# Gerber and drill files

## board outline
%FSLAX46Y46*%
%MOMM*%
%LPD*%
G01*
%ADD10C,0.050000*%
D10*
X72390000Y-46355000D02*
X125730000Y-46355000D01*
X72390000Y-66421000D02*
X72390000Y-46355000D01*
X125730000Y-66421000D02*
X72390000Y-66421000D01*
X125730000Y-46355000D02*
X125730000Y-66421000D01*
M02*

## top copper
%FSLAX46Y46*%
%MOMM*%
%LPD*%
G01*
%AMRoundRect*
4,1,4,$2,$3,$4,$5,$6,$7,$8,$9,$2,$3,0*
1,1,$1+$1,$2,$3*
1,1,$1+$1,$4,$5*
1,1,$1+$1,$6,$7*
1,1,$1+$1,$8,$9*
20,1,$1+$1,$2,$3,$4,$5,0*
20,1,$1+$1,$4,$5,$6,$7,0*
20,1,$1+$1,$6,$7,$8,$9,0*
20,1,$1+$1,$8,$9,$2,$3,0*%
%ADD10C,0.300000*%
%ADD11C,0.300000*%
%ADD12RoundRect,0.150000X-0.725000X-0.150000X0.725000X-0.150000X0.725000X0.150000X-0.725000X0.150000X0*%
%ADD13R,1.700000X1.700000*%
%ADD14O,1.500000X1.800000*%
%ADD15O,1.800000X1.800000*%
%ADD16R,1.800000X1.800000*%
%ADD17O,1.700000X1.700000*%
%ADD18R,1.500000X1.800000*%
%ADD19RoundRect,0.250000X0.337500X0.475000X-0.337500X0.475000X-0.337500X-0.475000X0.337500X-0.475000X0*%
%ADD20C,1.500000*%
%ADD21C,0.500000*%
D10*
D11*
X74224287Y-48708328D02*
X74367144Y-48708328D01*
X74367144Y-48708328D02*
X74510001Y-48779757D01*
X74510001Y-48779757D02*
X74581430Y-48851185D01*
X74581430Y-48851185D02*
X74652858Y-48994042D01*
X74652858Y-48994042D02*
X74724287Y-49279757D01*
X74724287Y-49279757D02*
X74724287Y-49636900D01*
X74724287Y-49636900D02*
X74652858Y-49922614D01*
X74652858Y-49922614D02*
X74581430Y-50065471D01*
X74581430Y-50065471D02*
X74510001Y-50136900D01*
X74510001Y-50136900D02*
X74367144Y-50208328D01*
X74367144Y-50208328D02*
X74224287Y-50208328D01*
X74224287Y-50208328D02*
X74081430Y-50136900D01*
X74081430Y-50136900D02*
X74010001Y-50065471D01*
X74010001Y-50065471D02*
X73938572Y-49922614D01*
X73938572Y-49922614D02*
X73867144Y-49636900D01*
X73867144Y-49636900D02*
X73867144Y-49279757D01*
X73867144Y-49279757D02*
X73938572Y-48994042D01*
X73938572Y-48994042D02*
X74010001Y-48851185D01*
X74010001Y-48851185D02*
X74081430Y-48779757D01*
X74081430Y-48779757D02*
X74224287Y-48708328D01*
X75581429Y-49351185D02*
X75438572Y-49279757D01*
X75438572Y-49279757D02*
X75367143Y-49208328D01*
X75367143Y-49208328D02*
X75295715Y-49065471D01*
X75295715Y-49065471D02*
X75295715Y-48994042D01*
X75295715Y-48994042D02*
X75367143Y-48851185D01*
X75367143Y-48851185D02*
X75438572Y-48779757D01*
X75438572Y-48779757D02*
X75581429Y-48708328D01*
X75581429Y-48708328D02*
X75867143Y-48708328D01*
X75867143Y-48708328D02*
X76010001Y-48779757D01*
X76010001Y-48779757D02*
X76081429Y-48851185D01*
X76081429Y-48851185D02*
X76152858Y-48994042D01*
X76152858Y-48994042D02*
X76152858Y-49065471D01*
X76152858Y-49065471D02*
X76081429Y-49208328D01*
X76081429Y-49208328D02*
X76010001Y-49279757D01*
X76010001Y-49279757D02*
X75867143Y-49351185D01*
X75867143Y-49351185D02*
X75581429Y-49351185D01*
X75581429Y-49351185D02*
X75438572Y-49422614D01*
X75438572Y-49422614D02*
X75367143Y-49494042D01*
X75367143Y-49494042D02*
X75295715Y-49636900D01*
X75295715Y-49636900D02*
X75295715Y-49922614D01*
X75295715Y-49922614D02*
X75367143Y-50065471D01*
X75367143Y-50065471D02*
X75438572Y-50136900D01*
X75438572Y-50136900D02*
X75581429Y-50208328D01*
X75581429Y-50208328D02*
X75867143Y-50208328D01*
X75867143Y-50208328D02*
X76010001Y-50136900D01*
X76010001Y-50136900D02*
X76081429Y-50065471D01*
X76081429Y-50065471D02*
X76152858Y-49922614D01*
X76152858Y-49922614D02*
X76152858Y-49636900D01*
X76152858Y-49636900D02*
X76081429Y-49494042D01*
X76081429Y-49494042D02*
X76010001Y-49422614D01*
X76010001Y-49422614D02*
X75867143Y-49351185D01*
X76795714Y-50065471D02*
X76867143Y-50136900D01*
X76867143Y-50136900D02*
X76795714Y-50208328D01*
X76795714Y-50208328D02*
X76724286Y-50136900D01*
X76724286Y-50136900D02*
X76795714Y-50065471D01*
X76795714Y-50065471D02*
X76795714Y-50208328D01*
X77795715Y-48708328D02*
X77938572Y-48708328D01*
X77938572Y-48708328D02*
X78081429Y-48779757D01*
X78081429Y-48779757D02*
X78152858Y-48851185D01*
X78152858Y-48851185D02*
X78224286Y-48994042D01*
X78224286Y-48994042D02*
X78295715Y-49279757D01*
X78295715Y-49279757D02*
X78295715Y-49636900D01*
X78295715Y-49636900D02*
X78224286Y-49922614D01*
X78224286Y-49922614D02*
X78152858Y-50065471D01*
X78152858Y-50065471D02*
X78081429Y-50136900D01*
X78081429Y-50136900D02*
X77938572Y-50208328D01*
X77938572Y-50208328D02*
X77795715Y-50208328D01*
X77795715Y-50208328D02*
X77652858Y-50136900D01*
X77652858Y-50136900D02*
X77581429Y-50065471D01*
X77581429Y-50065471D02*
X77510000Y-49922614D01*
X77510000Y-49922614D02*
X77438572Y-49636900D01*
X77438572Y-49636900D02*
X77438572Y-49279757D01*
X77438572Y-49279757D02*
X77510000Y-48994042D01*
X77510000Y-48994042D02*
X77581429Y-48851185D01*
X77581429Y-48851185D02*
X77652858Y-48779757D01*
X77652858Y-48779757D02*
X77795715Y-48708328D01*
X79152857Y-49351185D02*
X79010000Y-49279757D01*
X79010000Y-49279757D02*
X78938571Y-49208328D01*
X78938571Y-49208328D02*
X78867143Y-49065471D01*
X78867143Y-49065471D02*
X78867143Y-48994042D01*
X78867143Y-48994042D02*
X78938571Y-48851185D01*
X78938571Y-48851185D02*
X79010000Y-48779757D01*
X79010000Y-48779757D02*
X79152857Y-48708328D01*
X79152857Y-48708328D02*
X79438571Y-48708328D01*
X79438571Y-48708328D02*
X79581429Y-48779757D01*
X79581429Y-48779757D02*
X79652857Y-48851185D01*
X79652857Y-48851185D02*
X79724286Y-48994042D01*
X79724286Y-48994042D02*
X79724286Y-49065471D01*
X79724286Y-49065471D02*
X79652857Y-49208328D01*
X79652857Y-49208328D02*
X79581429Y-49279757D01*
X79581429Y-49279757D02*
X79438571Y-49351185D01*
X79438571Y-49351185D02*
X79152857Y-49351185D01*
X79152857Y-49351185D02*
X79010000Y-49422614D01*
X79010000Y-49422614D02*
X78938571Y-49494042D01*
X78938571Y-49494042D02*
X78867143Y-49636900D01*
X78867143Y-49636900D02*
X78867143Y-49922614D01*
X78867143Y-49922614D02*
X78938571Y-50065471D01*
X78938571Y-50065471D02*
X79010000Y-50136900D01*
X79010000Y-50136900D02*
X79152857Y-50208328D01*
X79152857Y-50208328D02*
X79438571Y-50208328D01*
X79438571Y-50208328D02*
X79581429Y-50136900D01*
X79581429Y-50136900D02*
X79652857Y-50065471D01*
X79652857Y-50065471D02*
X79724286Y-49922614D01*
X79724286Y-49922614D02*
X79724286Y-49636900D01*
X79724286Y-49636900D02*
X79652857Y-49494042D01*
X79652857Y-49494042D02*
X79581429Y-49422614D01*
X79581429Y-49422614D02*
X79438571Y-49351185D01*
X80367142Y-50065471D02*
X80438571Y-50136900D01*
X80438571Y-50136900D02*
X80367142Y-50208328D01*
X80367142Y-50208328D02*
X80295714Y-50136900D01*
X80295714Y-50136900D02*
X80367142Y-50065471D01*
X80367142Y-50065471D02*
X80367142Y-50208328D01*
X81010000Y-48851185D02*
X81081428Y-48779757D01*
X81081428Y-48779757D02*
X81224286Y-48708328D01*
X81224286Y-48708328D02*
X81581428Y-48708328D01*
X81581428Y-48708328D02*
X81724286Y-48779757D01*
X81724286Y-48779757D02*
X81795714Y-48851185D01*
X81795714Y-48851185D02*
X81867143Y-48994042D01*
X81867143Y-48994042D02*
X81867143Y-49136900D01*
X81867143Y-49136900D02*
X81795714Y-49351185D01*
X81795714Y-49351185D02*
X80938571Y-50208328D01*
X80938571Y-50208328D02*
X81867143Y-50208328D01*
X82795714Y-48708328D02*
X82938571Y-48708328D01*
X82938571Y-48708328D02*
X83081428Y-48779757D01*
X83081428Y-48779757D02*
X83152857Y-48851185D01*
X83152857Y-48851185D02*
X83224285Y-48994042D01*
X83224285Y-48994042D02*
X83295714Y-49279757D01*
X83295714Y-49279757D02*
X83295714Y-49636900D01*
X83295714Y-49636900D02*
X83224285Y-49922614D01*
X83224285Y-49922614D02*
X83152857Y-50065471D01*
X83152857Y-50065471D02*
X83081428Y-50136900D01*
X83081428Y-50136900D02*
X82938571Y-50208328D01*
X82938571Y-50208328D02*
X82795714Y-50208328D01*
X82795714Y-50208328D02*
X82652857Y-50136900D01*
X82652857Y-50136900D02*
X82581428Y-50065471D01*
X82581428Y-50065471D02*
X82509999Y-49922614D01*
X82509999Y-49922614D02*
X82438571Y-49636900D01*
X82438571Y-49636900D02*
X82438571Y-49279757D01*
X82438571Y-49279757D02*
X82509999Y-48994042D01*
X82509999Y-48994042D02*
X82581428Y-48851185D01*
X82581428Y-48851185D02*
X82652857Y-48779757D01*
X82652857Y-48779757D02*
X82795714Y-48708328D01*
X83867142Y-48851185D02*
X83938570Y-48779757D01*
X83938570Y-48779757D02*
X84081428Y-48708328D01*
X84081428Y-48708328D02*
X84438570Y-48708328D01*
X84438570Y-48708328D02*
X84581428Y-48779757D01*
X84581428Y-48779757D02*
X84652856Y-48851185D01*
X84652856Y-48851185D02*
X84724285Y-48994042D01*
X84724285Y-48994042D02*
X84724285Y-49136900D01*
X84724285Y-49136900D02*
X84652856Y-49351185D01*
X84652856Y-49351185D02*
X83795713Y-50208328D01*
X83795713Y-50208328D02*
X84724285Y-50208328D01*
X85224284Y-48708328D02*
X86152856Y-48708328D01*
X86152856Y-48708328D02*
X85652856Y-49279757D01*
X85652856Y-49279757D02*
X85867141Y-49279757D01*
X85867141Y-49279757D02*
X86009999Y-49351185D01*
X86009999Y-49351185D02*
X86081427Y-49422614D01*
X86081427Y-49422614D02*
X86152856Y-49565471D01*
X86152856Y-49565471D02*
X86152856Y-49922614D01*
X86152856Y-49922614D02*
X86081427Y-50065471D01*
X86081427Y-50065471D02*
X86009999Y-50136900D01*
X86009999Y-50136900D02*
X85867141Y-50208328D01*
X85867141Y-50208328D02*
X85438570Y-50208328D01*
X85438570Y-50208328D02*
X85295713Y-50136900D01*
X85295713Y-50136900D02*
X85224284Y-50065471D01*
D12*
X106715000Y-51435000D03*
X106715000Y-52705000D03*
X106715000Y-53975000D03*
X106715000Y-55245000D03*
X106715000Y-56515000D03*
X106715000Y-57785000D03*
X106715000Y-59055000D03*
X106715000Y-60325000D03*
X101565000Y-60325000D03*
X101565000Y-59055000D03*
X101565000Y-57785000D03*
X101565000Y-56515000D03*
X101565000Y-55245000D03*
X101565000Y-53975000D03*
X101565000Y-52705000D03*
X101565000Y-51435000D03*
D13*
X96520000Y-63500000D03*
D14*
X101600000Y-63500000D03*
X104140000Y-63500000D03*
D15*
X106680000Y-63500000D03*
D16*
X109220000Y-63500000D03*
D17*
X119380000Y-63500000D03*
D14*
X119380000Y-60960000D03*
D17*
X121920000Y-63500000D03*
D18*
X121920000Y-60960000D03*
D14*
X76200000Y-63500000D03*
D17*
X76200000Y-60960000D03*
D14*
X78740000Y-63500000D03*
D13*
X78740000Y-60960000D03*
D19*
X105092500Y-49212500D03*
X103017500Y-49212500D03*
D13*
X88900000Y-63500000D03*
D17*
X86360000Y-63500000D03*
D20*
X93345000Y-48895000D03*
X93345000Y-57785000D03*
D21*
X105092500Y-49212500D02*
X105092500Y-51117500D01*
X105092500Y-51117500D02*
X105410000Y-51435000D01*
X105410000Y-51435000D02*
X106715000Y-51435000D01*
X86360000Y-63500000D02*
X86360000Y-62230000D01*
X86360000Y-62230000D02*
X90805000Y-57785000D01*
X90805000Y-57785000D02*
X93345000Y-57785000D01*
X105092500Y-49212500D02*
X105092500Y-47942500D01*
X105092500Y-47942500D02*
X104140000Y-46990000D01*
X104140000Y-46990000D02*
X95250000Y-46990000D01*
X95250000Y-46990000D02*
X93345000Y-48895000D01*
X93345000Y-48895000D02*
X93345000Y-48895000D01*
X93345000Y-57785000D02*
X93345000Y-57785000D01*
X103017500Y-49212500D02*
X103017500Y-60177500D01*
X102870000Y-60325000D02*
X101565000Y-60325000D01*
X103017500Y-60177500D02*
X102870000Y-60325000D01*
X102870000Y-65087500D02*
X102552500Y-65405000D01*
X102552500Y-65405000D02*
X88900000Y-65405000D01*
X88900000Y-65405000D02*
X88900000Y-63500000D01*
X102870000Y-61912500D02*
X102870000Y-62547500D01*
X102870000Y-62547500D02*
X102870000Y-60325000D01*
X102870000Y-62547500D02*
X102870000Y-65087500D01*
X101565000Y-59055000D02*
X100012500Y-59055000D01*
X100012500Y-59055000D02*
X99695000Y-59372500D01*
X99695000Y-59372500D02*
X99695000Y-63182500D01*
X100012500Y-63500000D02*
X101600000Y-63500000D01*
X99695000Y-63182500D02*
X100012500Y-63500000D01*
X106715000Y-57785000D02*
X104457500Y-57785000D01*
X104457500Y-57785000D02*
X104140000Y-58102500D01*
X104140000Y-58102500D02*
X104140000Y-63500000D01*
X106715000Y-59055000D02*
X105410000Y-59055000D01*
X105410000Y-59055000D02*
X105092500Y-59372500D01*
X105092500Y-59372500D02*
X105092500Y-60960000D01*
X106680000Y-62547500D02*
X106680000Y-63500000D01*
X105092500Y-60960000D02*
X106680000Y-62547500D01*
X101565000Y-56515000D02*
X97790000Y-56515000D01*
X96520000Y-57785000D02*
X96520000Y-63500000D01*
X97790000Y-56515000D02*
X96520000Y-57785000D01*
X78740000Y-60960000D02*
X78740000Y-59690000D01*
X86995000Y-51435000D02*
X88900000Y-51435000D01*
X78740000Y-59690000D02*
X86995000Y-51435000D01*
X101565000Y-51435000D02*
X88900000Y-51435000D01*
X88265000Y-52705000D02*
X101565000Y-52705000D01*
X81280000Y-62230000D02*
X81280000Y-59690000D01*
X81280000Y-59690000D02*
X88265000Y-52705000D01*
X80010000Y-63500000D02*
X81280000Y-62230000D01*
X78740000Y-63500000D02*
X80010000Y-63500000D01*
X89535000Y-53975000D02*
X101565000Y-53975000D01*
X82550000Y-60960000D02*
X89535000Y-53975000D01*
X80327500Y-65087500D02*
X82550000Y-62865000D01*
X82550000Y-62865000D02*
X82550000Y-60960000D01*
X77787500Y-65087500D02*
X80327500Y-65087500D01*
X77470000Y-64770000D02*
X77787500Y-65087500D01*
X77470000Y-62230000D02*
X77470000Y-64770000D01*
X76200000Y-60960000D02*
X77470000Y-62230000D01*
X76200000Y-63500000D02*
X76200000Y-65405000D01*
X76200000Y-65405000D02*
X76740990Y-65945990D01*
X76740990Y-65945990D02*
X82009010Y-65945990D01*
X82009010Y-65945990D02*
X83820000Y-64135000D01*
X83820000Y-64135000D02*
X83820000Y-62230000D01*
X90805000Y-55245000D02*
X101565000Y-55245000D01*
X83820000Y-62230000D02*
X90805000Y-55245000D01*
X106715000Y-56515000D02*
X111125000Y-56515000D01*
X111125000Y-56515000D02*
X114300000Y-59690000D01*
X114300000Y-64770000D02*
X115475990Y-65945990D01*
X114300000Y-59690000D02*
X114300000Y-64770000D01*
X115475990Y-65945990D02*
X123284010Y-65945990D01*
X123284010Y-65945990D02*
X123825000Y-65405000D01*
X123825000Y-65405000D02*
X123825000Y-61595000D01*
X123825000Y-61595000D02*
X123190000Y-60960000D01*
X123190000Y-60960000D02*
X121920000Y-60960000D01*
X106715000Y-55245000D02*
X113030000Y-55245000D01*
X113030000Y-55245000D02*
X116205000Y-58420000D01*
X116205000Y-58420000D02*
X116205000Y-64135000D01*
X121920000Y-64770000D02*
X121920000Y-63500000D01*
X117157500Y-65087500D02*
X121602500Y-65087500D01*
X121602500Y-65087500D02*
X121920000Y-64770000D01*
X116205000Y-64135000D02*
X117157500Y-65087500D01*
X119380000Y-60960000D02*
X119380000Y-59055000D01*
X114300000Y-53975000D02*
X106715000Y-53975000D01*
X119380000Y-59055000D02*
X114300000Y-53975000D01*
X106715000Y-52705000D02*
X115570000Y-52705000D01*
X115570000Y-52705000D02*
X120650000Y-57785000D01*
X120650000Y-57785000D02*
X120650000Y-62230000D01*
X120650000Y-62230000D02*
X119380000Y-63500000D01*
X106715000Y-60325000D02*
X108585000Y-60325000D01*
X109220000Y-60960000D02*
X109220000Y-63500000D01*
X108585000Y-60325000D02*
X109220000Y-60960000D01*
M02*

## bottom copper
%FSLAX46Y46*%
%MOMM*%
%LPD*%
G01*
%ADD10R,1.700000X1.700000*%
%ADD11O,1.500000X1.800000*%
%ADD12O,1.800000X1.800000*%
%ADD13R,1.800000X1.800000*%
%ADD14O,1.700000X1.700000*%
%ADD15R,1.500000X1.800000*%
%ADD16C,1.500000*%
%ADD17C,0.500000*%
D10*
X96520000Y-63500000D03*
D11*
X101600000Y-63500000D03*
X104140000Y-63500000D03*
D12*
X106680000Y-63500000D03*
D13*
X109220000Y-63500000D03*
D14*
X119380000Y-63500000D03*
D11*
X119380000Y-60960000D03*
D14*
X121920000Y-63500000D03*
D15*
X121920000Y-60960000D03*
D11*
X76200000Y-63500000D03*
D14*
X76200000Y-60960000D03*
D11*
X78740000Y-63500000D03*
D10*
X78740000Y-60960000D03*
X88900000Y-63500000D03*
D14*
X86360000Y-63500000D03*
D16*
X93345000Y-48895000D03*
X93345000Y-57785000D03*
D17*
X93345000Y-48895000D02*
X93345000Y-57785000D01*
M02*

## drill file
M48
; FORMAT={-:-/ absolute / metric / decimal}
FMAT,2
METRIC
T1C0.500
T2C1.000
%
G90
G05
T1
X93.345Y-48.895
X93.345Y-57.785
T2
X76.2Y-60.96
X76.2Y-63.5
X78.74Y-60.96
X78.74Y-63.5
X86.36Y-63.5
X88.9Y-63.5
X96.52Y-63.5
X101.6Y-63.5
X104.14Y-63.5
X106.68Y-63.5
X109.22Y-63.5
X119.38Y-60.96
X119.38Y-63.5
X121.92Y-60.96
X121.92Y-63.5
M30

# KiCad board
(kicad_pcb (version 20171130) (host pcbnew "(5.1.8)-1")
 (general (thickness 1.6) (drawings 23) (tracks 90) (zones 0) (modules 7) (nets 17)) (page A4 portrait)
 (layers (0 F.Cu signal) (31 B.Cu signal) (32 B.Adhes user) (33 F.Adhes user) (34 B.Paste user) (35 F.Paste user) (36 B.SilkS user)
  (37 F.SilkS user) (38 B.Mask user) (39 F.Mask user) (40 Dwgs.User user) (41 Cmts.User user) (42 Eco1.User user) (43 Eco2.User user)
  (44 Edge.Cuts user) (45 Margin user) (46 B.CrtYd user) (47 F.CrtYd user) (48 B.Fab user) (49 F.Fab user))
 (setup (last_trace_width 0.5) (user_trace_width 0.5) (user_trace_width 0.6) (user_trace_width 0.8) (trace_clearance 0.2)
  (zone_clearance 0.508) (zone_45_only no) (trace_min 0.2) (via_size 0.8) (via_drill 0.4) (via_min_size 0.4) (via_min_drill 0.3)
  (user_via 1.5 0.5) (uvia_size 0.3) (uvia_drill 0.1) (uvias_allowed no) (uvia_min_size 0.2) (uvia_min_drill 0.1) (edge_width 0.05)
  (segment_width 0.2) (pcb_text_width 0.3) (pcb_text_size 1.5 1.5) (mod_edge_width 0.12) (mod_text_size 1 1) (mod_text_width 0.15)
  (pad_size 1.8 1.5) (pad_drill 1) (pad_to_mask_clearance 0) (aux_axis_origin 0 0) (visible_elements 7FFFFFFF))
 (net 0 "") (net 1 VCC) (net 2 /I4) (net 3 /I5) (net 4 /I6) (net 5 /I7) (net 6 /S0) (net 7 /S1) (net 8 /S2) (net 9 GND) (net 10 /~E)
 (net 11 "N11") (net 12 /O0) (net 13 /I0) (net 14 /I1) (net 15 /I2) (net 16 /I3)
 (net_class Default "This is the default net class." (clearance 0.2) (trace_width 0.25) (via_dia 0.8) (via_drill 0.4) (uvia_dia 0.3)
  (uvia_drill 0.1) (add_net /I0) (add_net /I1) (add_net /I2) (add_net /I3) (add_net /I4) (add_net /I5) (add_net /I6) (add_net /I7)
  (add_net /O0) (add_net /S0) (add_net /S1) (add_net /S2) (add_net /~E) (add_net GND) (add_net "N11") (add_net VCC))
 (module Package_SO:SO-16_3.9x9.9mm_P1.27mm (layer F.Cu) (at 104.14 55.88)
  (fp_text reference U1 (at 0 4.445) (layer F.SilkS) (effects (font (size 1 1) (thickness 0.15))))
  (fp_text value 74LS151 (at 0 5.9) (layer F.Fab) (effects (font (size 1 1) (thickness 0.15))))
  (pad 16 smd roundrect (at 2.575 -4.445) (size 1.75 0.6) (layers F.Cu F.Paste F.Mask) (roundrect_rratio 0.25) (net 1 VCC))
  (pad 15 smd roundrect (at 2.575 -3.175) (size 1.75 0.6) (layers F.Cu F.Paste F.Mask) (roundrect_rratio 0.25) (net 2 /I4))
  (pad 14 smd roundrect (at 2.575 -1.905) (size 1.75 0.6) (layers F.Cu F.Paste F.Mask) (roundrect_rratio 0.25) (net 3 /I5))
  (pad 13 smd roundrect (at 2.575 -0.635) (size 1.75 0.6) (layers F.Cu F.Paste F.Mask) (roundrect_rratio 0.25) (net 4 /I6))
  (pad 12 smd roundrect (at 2.575 0.635) (size 1.75 0.6) (layers F.Cu F.Paste F.Mask) (roundrect_rratio 0.25) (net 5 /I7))
  (pad 11 smd roundrect (at 2.575 1.905) (size 1.75 0.6) (layers F.Cu F.Paste F.Mask) (roundrect_rratio 0.25) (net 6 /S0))
  (pad 10 smd roundrect (at 2.575 3.175) (size 1.75 0.6) (layers F.Cu F.Paste F.Mask) (roundrect_rratio 0.25) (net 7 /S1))
  (pad 9 smd roundrect (at 2.575 4.445) (size 1.75 0.6) (layers F.Cu F.Paste F.Mask) (roundrect_rratio 0.25) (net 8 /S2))
  (pad 8 smd roundrect (at -2.575 4.445) (size 1.75 0.6) (layers F.Cu F.Paste F.Mask) (roundrect_rratio 0.25) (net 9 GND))
  (pad 7 smd roundrect (at -2.575 3.175) (size 1.75 0.6) (layers F.Cu F.Paste F.Mask) (roundrect_rratio 0.25) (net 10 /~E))
  (pad 6 smd roundrect (at -2.575 1.905) (size 1.75 0.6) (layers F.Cu F.Paste F.Mask) (roundrect_rratio 0.25) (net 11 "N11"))
  (pad 5 smd roundrect (at -2.575 0.635) (size 1.75 0.6) (layers F.Cu F.Paste F.Mask) (roundrect_rratio 0.25) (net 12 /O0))
  (pad 4 smd roundrect (at -2.575 -0.635) (size 1.75 0.6) (layers F.Cu F.Paste F.Mask) (roundrect_rratio 0.25) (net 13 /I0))
  (pad 3 smd roundrect (at -2.575 -1.905) (size 1.75 0.6) (layers F.Cu F.Paste F.Mask) (roundrect_rratio 0.25) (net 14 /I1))
  (pad 2 smd roundrect (at -2.575 -3.175) (size 1.75 0.6) (layers F.Cu F.Paste F.Mask) (roundrect_rratio 0.25) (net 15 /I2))
  (pad 1 smd roundrect (at -2.575 -4.445) (size 1.75 0.6) (layers F.Cu F.Paste F.Mask) (roundrect_rratio 0.25) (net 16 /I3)))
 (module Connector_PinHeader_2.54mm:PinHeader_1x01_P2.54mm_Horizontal (layer F.Cu) (at 96.52 63.5 270)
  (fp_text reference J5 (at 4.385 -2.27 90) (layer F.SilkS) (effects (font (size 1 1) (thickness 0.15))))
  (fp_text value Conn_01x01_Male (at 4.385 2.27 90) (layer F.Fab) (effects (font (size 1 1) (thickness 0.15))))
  (pad 1 thru_hole rect (at 0 0 270) (size 1.7 1.7) (drill 1) (layers *.Cu *.Mask) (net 12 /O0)))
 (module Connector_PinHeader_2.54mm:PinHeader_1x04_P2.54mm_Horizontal (layer F.Cu) (at 109.22 63.5 270)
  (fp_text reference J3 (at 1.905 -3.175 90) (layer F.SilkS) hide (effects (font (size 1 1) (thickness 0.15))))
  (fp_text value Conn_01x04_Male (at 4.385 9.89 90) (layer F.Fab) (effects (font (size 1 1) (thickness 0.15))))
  (pad 4 thru_hole oval (at 0 7.62 270) (size 1.8 1.5) (drill 1) (layers *.Cu *.Mask) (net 10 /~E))
  (pad 3 thru_hole oval (at 0 5.08 270) (size 1.8 1.5) (drill 1) (layers *.Cu *.Mask) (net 6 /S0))
  (pad 2 thru_hole oval (at 0 2.54 270) (size 1.8 1.8) (drill 1) (layers *.Cu *.Mask) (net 7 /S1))
  (pad 1 thru_hole rect (at 0 0 270) (size 1.8 1.8) (drill 1) (layers *.Cu *.Mask) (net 8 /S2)))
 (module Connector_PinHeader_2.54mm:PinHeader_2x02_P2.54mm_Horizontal (layer F.Cu) (at 121.92 60.96 270)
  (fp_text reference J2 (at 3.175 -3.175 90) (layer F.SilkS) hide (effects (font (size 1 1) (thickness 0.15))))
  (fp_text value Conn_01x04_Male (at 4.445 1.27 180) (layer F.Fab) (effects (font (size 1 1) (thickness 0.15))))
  (pad 4 thru_hole oval (at 2.54 2.54 270) (size 1.7 1.7) (drill 1) (layers *.Cu *.Mask) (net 2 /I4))
  (pad 3 thru_hole oval (at 0 2.54 270) (size 1.8 1.5) (drill 1) (layers *.Cu *.Mask) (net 3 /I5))
  (pad 2 thru_hole oval (at 2.54 0 270) (size 1.7 1.7) (drill 1) (layers *.Cu *.Mask) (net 4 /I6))
  (pad 1 thru_hole rect (at 0 0 270) (size 1.8 1.5) (drill 1) (layers *.Cu *.Mask) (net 5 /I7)))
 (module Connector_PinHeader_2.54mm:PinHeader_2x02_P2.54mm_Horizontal (layer F.Cu) (at 78.74 60.96 270)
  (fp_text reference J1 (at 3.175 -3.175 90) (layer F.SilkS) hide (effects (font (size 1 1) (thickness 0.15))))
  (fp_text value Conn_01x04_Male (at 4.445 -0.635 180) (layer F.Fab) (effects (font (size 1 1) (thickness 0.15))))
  (pad 4 thru_hole oval (at 2.54 2.54 270) (size 1.8 1.5) (drill 1) (layers *.Cu *.Mask) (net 13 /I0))
  (pad 3 thru_hole oval (at 0 2.54 270) (size 1.7 1.7) (drill 1) (layers *.Cu *.Mask) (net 14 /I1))
  (pad 2 thru_hole oval (at 2.54 0 270) (size 1.8 1.5) (drill 1) (layers *.Cu *.Mask) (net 15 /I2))
  (pad 1 thru_hole rect (at 0 0 270) (size 1.7 1.7) (drill 1) (layers *.Cu *.Mask) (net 16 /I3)))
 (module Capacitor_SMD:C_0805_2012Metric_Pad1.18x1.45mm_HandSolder (layer F.Cu) (at 104.055 49.2125 180)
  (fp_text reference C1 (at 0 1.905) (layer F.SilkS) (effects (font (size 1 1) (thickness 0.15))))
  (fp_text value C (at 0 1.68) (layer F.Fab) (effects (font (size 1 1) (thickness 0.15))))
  (pad 1 smd roundrect (at -1.0375 0 180) (size 1.175 1.45) (layers F.Cu F.Paste F.Mask) (roundrect_rratio 0.2127659574468085) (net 1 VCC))
  (pad 2 smd roundrect (at 1.0375 0 180) (size 1.175 1.45) (layers F.Cu F.Paste F.Mask) (roundrect_rratio 0.2127659574468085) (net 9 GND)))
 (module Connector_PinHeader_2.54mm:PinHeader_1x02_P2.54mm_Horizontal (layer F.Cu) (at 88.9 63.5 270)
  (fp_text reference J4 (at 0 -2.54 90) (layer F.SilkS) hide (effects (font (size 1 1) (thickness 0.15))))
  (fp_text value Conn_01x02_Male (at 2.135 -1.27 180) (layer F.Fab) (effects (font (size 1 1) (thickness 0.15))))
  (pad 1 thru_hole rect (at 0 0 270) (size 1.7 1.7) (drill 1) (layers *.Cu *.Mask) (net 9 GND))
  (pad 2 thru_hole oval (at 0 2.54 270) (size 1.7 1.7) (drill 1) (layers *.Cu *.Mask) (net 1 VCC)))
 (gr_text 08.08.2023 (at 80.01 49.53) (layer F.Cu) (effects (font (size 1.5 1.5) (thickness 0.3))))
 (gr_line (start 72.39 46.355) (end 125.73 46.355) (layer Edge.Cuts) (width 0.05))
 (gr_line (start 72.39 66.421) (end 72.39 46.355) (layer Edge.Cuts) (width 0.05))
 (gr_line (start 125.73 66.421) (end 72.39 66.421) (layer Edge.Cuts) (width 0.05))
 (gr_line (start 125.73 46.355) (end 125.73 66.421) (layer Edge.Cuts) (width 0.05))
 (segment (start 105.0925 49.2125) (end 105.0925 51.1175) (width 0.5) (layer F.Cu) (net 1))
 (segment (start 105.0925 51.1175) (end 105.41 51.435) (width 0.5) (layer F.Cu) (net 1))
 (segment (start 105.41 51.435) (end 106.715 51.435) (width 0.5) (layer F.Cu) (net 1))
 (segment (start 86.36 63.5) (end 86.36 62.23) (width 0.5) (layer F.Cu) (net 1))
 (segment (start 86.36 62.23) (end 90.805 57.785) (width 0.5) (layer F.Cu) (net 1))
 (segment (start 90.805 57.785) (end 93.345 57.785) (width 0.5) (layer F.Cu) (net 1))
 (segment (start 105.0925 49.2125) (end 105.0925 47.9425) (width 0.5) (layer F.Cu) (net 1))
 (segment (start 105.0925 47.9425) (end 104.14 46.99) (width 0.5) (layer F.Cu) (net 1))
 (segment (start 104.14 46.99) (end 95.25 46.99) (width 0.5) (layer F.Cu) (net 1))
 (segment (start 95.25 46.99) (end 93.345 48.895) (width 0.5) (layer F.Cu) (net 1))
 (segment (start 93.345 48.895) (end 93.345 48.895) (width 0.5) (layer F.Cu) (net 1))
 (via (at 93.345 48.895) (size 1.5) (drill 0.5) (layers F.Cu B.Cu) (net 1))
 (segment (start 93.345 57.785) (end 93.345 57.785) (width 0.5) (layer F.Cu) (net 1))
 (via (at 93.345 57.785) (size 1.5) (drill 0.5) (layers F.Cu B.Cu) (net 1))
 (segment (start 93.345 48.895) (end 93.345 57.785) (width 0.5) (layer B.Cu) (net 1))
 (segment (start 103.0175 49.2125) (end 103.0175 60.1775) (width 0.5) (layer F.Cu) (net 9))
 (segment (start 102.87 60.325) (end 101.565 60.325) (width 0.5) (layer F.Cu) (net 9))
 (segment (start 103.0175 60.1775) (end 102.87 60.325) (width 0.5) (layer F.Cu) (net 9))
 (segment (start 102.87 65.0875) (end 102.5525 65.405) (width 0.5) (layer F.Cu) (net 9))
 (segment (start 102.5525 65.405) (end 88.9 65.405) (width 0.5) (layer F.Cu) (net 9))
 (segment (start 88.9 65.405) (end 88.9 63.5) (width 0.5) (layer F.Cu) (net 9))
 (segment (start 102.87 61.9125) (end 102.87 62.5475) (width 0.5) (layer F.Cu) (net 9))
 (segment (start 102.87 62.5475) (end 102.87 60.325) (width 0.5) (layer F.Cu) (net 9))
 (segment (start 102.87 62.5475) (end 102.87 65.0875) (width 0.5) (layer F.Cu) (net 9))
 (segment (start 101.565 59.055) (end 100.0125 59.055) (width 0.5) (layer F.Cu) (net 10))
 (segment (start 100.0125 59.055) (end 99.695 59.3725) (width 0.5) (layer F.Cu) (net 10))
 (segment (start 99.695 59.3725) (end 99.695 63.1825) (width 0.5) (layer F.Cu) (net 10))
 (segment (start 100.0125 63.5) (end 101.6 63.5) (width 0.5) (layer F.Cu) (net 10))
 (segment (start 99.695 63.1825) (end 100.0125 63.5) (width 0.5) (layer F.Cu) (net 10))
 (segment (start 106.715 57.785) (end 104.4575 57.785) (width 0.5) (layer F.Cu) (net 6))
 (segment (start 104.4575 57.785) (end 104.14 58.1025) (width 0.5) (layer F.Cu) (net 6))
 (segment (start 104.14 58.1025) (end 104.14 63.5) (width 0.5) (layer F.Cu) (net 6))
 (segment (start 106.715 59.055) (end 105.41 59.055) (width 0.5) (layer F.Cu) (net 7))
 (segment (start 105.41 59.055) (end 105.0925 59.3725) (width 0.5) (layer F.Cu) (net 7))
 (segment (start 105.0925 59.3725) (end 105.0925 60.96) (width 0.5) (layer F.Cu) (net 7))
 (segment (start 106.68 62.5475) (end 106.68 63.5) (width 0.5) (layer F.Cu) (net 7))
 (segment (start 105.0925 60.96) (end 106.68 62.5475) (width 0.5) (layer F.Cu) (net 7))
 (segment (start 101.565 56.515) (end 97.79 56.515) (width 0.5) (layer F.Cu) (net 12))
 (segment (start 96.52 57.785) (end 96.52 63.5) (width 0.5) (layer F.Cu) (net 12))
 (segment (start 97.79 56.515) (end 96.52 57.785) (width 0.5) (layer F.Cu) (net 12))
 (segment (start 78.74 60.96) (end 78.74 59.69) (width 0.5) (layer F.Cu) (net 16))
 (segment (start 86.995 51.435) (end 88.9 51.435) (width 0.5) (layer F.Cu) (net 16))
 (segment (start 78.74 59.69) (end 86.995 51.435) (width 0.5) (layer F.Cu) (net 16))
 (segment (start 101.565 51.435) (end 88.9 51.435) (width 0.5) (layer F.Cu) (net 16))
 (segment (start 88.265 52.705) (end 101.565 52.705) (width 0.5) (layer F.Cu) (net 15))
 (segment (start 81.28 62.23) (end 81.28 59.69) (width 0.5) (layer F.Cu) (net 15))
 (segment (start 81.28 59.69) (end 88.265 52.705) (width 0.5) (layer F.Cu) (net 15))
 (segment (start 80.01 63.5) (end 81.28 62.23) (width 0.5) (layer F.Cu) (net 15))
 (segment (start 78.74 63.5) (end 80.01 63.5) (width 0.5) (layer F.Cu) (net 15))
 (segment (start 89.535 53.975) (end 101.565 53.975) (width 0.5) (layer F.Cu) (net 14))
 (segment (start 82.55 60.96) (end 89.535 53.975) (width 0.5) (layer F.Cu) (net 14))
 (segment (start 80.3275 65.0875) (end 82.55 62.865) (width 0.5) (layer F.Cu) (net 14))
 (segment (start 82.55 62.865) (end 82.55 60.96) (width 0.5) (layer F.Cu) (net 14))
 (segment (start 77.7875 65.0875) (end 80.3275 65.0875) (width 0.5) (layer F.Cu) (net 14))
 (segment (start 77.47 64.77) (end 77.7875 65.0875) (width 0.5) (layer F.Cu) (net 14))
 (segment (start 77.47 62.23) (end 77.47 64.77) (width 0.5) (layer F.Cu) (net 14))
 (segment (start 76.2 60.96) (end 77.47 62.23) (width 0.5) (layer F.Cu) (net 14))
 (segment (start 76.2 63.5) (end 76.2 65.405) (width 0.5) (layer F.Cu) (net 13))
 (segment (start 76.2 65.405) (end 76.74099 65.94599) (width 0.5) (layer F.Cu) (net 13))
 (segment (start 76.74099 65.94599) (end 82.00901 65.94599) (width 0.5) (layer F.Cu) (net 13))
 (segment (start 82.00901 65.94599) (end 83.82 64.135) (width 0.5) (layer F.Cu) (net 13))
 (segment (start 83.82 64.135) (end 83.82 62.23) (width 0.5) (layer F.Cu) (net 13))
 (segment (start 90.805 55.245) (end 101.565 55.245) (width 0.5) (layer F.Cu) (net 13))
 (segment (start 83.82 62.23) (end 90.805 55.245) (width 0.5) (layer F.Cu) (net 13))
 (segment (start 106.715 56.515) (end 111.125 56.515) (width 0.5) (layer F.Cu) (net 5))
 (segment (start 111.125 56.515) (end 114.3 59.69) (width 0.5) (layer F.Cu) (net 5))
 (segment (start 114.3 64.77) (end 115.47599 65.94599) (width 0.5) (layer F.Cu) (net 5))
 (segment (start 114.3 59.69) (end 114.3 64.77) (width 0.5) (layer F.Cu) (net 5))
 (segment (start 115.47599 65.94599) (end 123.28401 65.94599) (width 0.5) (layer F.Cu) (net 5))
 (segment (start 123.28401 65.94599) (end 123.825 65.405) (width 0.5) (layer F.Cu) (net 5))
 (segment (start 123.825 65.405) (end 123.825 61.595) (width 0.5) (layer F.Cu) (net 5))
 (segment (start 123.825 61.595) (end 123.19 60.96) (width 0.5) (layer F.Cu) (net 5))
 (segment (start 123.19 60.96) (end 121.92 60.96) (width 0.5) (layer F.Cu) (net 5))
 (segment (start 106.715 55.245) (end 113.03 55.245) (width 0.5) (layer F.Cu) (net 4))
 (segment (start 113.03 55.245) (end 116.205 58.42) (width 0.5) (layer F.Cu) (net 4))
 (segment (start 116.205 58.42) (end 116.205 64.135) (width 0.5) (layer F.Cu) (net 4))
 (segment (start 121.92 64.77) (end 121.92 63.5) (width 0.5) (layer F.Cu) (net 4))
 (segment (start 117.1575 65.0875) (end 121.6025 65.0875) (width 0.5) (layer F.Cu) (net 4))
 (segment (start 121.6025 65.0875) (end 121.92 64.77) (width 0.5) (layer F.Cu) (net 4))
 (segment (start 116.205 64.135) (end 117.1575 65.0875) (width 0.5) (layer F.Cu) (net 4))
 (segment (start 119.38 60.96) (end 119.38 59.055) (width 0.5) (layer F.Cu) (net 3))
 (segment (start 114.3 53.975) (end 106.715 53.975) (width 0.5) (layer F.Cu) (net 3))
 (segment (start 119.38 59.055) (end 114.3 53.975) (width 0.5) (layer F.Cu) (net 3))
 (segment (start 106.715 52.705) (end 115.57 52.705) (width 0.5) (layer F.Cu) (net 2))
 (segment (start 115.57 52.705) (end 120.65 57.785) (width 0.5) (layer F.Cu) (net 2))
 (segment (start 120.65 57.785) (end 120.65 62.23) (width 0.5) (layer F.Cu) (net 2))
 (segment (start 120.65 62.23) (end 119.38 63.5) (width 0.5) (layer F.Cu) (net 2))
 (segment (start 106.715 60.325) (end 108.585 60.325) (width 0.5) (layer F.Cu) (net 8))
 (segment (start 109.22 60.96) (end 109.22 63.5) (width 0.5) (layer F.Cu) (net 8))
 (segment (start 108.585 60.325) (end 109.22 60.96) (width 0.5) (layer F.Cu) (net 8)))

